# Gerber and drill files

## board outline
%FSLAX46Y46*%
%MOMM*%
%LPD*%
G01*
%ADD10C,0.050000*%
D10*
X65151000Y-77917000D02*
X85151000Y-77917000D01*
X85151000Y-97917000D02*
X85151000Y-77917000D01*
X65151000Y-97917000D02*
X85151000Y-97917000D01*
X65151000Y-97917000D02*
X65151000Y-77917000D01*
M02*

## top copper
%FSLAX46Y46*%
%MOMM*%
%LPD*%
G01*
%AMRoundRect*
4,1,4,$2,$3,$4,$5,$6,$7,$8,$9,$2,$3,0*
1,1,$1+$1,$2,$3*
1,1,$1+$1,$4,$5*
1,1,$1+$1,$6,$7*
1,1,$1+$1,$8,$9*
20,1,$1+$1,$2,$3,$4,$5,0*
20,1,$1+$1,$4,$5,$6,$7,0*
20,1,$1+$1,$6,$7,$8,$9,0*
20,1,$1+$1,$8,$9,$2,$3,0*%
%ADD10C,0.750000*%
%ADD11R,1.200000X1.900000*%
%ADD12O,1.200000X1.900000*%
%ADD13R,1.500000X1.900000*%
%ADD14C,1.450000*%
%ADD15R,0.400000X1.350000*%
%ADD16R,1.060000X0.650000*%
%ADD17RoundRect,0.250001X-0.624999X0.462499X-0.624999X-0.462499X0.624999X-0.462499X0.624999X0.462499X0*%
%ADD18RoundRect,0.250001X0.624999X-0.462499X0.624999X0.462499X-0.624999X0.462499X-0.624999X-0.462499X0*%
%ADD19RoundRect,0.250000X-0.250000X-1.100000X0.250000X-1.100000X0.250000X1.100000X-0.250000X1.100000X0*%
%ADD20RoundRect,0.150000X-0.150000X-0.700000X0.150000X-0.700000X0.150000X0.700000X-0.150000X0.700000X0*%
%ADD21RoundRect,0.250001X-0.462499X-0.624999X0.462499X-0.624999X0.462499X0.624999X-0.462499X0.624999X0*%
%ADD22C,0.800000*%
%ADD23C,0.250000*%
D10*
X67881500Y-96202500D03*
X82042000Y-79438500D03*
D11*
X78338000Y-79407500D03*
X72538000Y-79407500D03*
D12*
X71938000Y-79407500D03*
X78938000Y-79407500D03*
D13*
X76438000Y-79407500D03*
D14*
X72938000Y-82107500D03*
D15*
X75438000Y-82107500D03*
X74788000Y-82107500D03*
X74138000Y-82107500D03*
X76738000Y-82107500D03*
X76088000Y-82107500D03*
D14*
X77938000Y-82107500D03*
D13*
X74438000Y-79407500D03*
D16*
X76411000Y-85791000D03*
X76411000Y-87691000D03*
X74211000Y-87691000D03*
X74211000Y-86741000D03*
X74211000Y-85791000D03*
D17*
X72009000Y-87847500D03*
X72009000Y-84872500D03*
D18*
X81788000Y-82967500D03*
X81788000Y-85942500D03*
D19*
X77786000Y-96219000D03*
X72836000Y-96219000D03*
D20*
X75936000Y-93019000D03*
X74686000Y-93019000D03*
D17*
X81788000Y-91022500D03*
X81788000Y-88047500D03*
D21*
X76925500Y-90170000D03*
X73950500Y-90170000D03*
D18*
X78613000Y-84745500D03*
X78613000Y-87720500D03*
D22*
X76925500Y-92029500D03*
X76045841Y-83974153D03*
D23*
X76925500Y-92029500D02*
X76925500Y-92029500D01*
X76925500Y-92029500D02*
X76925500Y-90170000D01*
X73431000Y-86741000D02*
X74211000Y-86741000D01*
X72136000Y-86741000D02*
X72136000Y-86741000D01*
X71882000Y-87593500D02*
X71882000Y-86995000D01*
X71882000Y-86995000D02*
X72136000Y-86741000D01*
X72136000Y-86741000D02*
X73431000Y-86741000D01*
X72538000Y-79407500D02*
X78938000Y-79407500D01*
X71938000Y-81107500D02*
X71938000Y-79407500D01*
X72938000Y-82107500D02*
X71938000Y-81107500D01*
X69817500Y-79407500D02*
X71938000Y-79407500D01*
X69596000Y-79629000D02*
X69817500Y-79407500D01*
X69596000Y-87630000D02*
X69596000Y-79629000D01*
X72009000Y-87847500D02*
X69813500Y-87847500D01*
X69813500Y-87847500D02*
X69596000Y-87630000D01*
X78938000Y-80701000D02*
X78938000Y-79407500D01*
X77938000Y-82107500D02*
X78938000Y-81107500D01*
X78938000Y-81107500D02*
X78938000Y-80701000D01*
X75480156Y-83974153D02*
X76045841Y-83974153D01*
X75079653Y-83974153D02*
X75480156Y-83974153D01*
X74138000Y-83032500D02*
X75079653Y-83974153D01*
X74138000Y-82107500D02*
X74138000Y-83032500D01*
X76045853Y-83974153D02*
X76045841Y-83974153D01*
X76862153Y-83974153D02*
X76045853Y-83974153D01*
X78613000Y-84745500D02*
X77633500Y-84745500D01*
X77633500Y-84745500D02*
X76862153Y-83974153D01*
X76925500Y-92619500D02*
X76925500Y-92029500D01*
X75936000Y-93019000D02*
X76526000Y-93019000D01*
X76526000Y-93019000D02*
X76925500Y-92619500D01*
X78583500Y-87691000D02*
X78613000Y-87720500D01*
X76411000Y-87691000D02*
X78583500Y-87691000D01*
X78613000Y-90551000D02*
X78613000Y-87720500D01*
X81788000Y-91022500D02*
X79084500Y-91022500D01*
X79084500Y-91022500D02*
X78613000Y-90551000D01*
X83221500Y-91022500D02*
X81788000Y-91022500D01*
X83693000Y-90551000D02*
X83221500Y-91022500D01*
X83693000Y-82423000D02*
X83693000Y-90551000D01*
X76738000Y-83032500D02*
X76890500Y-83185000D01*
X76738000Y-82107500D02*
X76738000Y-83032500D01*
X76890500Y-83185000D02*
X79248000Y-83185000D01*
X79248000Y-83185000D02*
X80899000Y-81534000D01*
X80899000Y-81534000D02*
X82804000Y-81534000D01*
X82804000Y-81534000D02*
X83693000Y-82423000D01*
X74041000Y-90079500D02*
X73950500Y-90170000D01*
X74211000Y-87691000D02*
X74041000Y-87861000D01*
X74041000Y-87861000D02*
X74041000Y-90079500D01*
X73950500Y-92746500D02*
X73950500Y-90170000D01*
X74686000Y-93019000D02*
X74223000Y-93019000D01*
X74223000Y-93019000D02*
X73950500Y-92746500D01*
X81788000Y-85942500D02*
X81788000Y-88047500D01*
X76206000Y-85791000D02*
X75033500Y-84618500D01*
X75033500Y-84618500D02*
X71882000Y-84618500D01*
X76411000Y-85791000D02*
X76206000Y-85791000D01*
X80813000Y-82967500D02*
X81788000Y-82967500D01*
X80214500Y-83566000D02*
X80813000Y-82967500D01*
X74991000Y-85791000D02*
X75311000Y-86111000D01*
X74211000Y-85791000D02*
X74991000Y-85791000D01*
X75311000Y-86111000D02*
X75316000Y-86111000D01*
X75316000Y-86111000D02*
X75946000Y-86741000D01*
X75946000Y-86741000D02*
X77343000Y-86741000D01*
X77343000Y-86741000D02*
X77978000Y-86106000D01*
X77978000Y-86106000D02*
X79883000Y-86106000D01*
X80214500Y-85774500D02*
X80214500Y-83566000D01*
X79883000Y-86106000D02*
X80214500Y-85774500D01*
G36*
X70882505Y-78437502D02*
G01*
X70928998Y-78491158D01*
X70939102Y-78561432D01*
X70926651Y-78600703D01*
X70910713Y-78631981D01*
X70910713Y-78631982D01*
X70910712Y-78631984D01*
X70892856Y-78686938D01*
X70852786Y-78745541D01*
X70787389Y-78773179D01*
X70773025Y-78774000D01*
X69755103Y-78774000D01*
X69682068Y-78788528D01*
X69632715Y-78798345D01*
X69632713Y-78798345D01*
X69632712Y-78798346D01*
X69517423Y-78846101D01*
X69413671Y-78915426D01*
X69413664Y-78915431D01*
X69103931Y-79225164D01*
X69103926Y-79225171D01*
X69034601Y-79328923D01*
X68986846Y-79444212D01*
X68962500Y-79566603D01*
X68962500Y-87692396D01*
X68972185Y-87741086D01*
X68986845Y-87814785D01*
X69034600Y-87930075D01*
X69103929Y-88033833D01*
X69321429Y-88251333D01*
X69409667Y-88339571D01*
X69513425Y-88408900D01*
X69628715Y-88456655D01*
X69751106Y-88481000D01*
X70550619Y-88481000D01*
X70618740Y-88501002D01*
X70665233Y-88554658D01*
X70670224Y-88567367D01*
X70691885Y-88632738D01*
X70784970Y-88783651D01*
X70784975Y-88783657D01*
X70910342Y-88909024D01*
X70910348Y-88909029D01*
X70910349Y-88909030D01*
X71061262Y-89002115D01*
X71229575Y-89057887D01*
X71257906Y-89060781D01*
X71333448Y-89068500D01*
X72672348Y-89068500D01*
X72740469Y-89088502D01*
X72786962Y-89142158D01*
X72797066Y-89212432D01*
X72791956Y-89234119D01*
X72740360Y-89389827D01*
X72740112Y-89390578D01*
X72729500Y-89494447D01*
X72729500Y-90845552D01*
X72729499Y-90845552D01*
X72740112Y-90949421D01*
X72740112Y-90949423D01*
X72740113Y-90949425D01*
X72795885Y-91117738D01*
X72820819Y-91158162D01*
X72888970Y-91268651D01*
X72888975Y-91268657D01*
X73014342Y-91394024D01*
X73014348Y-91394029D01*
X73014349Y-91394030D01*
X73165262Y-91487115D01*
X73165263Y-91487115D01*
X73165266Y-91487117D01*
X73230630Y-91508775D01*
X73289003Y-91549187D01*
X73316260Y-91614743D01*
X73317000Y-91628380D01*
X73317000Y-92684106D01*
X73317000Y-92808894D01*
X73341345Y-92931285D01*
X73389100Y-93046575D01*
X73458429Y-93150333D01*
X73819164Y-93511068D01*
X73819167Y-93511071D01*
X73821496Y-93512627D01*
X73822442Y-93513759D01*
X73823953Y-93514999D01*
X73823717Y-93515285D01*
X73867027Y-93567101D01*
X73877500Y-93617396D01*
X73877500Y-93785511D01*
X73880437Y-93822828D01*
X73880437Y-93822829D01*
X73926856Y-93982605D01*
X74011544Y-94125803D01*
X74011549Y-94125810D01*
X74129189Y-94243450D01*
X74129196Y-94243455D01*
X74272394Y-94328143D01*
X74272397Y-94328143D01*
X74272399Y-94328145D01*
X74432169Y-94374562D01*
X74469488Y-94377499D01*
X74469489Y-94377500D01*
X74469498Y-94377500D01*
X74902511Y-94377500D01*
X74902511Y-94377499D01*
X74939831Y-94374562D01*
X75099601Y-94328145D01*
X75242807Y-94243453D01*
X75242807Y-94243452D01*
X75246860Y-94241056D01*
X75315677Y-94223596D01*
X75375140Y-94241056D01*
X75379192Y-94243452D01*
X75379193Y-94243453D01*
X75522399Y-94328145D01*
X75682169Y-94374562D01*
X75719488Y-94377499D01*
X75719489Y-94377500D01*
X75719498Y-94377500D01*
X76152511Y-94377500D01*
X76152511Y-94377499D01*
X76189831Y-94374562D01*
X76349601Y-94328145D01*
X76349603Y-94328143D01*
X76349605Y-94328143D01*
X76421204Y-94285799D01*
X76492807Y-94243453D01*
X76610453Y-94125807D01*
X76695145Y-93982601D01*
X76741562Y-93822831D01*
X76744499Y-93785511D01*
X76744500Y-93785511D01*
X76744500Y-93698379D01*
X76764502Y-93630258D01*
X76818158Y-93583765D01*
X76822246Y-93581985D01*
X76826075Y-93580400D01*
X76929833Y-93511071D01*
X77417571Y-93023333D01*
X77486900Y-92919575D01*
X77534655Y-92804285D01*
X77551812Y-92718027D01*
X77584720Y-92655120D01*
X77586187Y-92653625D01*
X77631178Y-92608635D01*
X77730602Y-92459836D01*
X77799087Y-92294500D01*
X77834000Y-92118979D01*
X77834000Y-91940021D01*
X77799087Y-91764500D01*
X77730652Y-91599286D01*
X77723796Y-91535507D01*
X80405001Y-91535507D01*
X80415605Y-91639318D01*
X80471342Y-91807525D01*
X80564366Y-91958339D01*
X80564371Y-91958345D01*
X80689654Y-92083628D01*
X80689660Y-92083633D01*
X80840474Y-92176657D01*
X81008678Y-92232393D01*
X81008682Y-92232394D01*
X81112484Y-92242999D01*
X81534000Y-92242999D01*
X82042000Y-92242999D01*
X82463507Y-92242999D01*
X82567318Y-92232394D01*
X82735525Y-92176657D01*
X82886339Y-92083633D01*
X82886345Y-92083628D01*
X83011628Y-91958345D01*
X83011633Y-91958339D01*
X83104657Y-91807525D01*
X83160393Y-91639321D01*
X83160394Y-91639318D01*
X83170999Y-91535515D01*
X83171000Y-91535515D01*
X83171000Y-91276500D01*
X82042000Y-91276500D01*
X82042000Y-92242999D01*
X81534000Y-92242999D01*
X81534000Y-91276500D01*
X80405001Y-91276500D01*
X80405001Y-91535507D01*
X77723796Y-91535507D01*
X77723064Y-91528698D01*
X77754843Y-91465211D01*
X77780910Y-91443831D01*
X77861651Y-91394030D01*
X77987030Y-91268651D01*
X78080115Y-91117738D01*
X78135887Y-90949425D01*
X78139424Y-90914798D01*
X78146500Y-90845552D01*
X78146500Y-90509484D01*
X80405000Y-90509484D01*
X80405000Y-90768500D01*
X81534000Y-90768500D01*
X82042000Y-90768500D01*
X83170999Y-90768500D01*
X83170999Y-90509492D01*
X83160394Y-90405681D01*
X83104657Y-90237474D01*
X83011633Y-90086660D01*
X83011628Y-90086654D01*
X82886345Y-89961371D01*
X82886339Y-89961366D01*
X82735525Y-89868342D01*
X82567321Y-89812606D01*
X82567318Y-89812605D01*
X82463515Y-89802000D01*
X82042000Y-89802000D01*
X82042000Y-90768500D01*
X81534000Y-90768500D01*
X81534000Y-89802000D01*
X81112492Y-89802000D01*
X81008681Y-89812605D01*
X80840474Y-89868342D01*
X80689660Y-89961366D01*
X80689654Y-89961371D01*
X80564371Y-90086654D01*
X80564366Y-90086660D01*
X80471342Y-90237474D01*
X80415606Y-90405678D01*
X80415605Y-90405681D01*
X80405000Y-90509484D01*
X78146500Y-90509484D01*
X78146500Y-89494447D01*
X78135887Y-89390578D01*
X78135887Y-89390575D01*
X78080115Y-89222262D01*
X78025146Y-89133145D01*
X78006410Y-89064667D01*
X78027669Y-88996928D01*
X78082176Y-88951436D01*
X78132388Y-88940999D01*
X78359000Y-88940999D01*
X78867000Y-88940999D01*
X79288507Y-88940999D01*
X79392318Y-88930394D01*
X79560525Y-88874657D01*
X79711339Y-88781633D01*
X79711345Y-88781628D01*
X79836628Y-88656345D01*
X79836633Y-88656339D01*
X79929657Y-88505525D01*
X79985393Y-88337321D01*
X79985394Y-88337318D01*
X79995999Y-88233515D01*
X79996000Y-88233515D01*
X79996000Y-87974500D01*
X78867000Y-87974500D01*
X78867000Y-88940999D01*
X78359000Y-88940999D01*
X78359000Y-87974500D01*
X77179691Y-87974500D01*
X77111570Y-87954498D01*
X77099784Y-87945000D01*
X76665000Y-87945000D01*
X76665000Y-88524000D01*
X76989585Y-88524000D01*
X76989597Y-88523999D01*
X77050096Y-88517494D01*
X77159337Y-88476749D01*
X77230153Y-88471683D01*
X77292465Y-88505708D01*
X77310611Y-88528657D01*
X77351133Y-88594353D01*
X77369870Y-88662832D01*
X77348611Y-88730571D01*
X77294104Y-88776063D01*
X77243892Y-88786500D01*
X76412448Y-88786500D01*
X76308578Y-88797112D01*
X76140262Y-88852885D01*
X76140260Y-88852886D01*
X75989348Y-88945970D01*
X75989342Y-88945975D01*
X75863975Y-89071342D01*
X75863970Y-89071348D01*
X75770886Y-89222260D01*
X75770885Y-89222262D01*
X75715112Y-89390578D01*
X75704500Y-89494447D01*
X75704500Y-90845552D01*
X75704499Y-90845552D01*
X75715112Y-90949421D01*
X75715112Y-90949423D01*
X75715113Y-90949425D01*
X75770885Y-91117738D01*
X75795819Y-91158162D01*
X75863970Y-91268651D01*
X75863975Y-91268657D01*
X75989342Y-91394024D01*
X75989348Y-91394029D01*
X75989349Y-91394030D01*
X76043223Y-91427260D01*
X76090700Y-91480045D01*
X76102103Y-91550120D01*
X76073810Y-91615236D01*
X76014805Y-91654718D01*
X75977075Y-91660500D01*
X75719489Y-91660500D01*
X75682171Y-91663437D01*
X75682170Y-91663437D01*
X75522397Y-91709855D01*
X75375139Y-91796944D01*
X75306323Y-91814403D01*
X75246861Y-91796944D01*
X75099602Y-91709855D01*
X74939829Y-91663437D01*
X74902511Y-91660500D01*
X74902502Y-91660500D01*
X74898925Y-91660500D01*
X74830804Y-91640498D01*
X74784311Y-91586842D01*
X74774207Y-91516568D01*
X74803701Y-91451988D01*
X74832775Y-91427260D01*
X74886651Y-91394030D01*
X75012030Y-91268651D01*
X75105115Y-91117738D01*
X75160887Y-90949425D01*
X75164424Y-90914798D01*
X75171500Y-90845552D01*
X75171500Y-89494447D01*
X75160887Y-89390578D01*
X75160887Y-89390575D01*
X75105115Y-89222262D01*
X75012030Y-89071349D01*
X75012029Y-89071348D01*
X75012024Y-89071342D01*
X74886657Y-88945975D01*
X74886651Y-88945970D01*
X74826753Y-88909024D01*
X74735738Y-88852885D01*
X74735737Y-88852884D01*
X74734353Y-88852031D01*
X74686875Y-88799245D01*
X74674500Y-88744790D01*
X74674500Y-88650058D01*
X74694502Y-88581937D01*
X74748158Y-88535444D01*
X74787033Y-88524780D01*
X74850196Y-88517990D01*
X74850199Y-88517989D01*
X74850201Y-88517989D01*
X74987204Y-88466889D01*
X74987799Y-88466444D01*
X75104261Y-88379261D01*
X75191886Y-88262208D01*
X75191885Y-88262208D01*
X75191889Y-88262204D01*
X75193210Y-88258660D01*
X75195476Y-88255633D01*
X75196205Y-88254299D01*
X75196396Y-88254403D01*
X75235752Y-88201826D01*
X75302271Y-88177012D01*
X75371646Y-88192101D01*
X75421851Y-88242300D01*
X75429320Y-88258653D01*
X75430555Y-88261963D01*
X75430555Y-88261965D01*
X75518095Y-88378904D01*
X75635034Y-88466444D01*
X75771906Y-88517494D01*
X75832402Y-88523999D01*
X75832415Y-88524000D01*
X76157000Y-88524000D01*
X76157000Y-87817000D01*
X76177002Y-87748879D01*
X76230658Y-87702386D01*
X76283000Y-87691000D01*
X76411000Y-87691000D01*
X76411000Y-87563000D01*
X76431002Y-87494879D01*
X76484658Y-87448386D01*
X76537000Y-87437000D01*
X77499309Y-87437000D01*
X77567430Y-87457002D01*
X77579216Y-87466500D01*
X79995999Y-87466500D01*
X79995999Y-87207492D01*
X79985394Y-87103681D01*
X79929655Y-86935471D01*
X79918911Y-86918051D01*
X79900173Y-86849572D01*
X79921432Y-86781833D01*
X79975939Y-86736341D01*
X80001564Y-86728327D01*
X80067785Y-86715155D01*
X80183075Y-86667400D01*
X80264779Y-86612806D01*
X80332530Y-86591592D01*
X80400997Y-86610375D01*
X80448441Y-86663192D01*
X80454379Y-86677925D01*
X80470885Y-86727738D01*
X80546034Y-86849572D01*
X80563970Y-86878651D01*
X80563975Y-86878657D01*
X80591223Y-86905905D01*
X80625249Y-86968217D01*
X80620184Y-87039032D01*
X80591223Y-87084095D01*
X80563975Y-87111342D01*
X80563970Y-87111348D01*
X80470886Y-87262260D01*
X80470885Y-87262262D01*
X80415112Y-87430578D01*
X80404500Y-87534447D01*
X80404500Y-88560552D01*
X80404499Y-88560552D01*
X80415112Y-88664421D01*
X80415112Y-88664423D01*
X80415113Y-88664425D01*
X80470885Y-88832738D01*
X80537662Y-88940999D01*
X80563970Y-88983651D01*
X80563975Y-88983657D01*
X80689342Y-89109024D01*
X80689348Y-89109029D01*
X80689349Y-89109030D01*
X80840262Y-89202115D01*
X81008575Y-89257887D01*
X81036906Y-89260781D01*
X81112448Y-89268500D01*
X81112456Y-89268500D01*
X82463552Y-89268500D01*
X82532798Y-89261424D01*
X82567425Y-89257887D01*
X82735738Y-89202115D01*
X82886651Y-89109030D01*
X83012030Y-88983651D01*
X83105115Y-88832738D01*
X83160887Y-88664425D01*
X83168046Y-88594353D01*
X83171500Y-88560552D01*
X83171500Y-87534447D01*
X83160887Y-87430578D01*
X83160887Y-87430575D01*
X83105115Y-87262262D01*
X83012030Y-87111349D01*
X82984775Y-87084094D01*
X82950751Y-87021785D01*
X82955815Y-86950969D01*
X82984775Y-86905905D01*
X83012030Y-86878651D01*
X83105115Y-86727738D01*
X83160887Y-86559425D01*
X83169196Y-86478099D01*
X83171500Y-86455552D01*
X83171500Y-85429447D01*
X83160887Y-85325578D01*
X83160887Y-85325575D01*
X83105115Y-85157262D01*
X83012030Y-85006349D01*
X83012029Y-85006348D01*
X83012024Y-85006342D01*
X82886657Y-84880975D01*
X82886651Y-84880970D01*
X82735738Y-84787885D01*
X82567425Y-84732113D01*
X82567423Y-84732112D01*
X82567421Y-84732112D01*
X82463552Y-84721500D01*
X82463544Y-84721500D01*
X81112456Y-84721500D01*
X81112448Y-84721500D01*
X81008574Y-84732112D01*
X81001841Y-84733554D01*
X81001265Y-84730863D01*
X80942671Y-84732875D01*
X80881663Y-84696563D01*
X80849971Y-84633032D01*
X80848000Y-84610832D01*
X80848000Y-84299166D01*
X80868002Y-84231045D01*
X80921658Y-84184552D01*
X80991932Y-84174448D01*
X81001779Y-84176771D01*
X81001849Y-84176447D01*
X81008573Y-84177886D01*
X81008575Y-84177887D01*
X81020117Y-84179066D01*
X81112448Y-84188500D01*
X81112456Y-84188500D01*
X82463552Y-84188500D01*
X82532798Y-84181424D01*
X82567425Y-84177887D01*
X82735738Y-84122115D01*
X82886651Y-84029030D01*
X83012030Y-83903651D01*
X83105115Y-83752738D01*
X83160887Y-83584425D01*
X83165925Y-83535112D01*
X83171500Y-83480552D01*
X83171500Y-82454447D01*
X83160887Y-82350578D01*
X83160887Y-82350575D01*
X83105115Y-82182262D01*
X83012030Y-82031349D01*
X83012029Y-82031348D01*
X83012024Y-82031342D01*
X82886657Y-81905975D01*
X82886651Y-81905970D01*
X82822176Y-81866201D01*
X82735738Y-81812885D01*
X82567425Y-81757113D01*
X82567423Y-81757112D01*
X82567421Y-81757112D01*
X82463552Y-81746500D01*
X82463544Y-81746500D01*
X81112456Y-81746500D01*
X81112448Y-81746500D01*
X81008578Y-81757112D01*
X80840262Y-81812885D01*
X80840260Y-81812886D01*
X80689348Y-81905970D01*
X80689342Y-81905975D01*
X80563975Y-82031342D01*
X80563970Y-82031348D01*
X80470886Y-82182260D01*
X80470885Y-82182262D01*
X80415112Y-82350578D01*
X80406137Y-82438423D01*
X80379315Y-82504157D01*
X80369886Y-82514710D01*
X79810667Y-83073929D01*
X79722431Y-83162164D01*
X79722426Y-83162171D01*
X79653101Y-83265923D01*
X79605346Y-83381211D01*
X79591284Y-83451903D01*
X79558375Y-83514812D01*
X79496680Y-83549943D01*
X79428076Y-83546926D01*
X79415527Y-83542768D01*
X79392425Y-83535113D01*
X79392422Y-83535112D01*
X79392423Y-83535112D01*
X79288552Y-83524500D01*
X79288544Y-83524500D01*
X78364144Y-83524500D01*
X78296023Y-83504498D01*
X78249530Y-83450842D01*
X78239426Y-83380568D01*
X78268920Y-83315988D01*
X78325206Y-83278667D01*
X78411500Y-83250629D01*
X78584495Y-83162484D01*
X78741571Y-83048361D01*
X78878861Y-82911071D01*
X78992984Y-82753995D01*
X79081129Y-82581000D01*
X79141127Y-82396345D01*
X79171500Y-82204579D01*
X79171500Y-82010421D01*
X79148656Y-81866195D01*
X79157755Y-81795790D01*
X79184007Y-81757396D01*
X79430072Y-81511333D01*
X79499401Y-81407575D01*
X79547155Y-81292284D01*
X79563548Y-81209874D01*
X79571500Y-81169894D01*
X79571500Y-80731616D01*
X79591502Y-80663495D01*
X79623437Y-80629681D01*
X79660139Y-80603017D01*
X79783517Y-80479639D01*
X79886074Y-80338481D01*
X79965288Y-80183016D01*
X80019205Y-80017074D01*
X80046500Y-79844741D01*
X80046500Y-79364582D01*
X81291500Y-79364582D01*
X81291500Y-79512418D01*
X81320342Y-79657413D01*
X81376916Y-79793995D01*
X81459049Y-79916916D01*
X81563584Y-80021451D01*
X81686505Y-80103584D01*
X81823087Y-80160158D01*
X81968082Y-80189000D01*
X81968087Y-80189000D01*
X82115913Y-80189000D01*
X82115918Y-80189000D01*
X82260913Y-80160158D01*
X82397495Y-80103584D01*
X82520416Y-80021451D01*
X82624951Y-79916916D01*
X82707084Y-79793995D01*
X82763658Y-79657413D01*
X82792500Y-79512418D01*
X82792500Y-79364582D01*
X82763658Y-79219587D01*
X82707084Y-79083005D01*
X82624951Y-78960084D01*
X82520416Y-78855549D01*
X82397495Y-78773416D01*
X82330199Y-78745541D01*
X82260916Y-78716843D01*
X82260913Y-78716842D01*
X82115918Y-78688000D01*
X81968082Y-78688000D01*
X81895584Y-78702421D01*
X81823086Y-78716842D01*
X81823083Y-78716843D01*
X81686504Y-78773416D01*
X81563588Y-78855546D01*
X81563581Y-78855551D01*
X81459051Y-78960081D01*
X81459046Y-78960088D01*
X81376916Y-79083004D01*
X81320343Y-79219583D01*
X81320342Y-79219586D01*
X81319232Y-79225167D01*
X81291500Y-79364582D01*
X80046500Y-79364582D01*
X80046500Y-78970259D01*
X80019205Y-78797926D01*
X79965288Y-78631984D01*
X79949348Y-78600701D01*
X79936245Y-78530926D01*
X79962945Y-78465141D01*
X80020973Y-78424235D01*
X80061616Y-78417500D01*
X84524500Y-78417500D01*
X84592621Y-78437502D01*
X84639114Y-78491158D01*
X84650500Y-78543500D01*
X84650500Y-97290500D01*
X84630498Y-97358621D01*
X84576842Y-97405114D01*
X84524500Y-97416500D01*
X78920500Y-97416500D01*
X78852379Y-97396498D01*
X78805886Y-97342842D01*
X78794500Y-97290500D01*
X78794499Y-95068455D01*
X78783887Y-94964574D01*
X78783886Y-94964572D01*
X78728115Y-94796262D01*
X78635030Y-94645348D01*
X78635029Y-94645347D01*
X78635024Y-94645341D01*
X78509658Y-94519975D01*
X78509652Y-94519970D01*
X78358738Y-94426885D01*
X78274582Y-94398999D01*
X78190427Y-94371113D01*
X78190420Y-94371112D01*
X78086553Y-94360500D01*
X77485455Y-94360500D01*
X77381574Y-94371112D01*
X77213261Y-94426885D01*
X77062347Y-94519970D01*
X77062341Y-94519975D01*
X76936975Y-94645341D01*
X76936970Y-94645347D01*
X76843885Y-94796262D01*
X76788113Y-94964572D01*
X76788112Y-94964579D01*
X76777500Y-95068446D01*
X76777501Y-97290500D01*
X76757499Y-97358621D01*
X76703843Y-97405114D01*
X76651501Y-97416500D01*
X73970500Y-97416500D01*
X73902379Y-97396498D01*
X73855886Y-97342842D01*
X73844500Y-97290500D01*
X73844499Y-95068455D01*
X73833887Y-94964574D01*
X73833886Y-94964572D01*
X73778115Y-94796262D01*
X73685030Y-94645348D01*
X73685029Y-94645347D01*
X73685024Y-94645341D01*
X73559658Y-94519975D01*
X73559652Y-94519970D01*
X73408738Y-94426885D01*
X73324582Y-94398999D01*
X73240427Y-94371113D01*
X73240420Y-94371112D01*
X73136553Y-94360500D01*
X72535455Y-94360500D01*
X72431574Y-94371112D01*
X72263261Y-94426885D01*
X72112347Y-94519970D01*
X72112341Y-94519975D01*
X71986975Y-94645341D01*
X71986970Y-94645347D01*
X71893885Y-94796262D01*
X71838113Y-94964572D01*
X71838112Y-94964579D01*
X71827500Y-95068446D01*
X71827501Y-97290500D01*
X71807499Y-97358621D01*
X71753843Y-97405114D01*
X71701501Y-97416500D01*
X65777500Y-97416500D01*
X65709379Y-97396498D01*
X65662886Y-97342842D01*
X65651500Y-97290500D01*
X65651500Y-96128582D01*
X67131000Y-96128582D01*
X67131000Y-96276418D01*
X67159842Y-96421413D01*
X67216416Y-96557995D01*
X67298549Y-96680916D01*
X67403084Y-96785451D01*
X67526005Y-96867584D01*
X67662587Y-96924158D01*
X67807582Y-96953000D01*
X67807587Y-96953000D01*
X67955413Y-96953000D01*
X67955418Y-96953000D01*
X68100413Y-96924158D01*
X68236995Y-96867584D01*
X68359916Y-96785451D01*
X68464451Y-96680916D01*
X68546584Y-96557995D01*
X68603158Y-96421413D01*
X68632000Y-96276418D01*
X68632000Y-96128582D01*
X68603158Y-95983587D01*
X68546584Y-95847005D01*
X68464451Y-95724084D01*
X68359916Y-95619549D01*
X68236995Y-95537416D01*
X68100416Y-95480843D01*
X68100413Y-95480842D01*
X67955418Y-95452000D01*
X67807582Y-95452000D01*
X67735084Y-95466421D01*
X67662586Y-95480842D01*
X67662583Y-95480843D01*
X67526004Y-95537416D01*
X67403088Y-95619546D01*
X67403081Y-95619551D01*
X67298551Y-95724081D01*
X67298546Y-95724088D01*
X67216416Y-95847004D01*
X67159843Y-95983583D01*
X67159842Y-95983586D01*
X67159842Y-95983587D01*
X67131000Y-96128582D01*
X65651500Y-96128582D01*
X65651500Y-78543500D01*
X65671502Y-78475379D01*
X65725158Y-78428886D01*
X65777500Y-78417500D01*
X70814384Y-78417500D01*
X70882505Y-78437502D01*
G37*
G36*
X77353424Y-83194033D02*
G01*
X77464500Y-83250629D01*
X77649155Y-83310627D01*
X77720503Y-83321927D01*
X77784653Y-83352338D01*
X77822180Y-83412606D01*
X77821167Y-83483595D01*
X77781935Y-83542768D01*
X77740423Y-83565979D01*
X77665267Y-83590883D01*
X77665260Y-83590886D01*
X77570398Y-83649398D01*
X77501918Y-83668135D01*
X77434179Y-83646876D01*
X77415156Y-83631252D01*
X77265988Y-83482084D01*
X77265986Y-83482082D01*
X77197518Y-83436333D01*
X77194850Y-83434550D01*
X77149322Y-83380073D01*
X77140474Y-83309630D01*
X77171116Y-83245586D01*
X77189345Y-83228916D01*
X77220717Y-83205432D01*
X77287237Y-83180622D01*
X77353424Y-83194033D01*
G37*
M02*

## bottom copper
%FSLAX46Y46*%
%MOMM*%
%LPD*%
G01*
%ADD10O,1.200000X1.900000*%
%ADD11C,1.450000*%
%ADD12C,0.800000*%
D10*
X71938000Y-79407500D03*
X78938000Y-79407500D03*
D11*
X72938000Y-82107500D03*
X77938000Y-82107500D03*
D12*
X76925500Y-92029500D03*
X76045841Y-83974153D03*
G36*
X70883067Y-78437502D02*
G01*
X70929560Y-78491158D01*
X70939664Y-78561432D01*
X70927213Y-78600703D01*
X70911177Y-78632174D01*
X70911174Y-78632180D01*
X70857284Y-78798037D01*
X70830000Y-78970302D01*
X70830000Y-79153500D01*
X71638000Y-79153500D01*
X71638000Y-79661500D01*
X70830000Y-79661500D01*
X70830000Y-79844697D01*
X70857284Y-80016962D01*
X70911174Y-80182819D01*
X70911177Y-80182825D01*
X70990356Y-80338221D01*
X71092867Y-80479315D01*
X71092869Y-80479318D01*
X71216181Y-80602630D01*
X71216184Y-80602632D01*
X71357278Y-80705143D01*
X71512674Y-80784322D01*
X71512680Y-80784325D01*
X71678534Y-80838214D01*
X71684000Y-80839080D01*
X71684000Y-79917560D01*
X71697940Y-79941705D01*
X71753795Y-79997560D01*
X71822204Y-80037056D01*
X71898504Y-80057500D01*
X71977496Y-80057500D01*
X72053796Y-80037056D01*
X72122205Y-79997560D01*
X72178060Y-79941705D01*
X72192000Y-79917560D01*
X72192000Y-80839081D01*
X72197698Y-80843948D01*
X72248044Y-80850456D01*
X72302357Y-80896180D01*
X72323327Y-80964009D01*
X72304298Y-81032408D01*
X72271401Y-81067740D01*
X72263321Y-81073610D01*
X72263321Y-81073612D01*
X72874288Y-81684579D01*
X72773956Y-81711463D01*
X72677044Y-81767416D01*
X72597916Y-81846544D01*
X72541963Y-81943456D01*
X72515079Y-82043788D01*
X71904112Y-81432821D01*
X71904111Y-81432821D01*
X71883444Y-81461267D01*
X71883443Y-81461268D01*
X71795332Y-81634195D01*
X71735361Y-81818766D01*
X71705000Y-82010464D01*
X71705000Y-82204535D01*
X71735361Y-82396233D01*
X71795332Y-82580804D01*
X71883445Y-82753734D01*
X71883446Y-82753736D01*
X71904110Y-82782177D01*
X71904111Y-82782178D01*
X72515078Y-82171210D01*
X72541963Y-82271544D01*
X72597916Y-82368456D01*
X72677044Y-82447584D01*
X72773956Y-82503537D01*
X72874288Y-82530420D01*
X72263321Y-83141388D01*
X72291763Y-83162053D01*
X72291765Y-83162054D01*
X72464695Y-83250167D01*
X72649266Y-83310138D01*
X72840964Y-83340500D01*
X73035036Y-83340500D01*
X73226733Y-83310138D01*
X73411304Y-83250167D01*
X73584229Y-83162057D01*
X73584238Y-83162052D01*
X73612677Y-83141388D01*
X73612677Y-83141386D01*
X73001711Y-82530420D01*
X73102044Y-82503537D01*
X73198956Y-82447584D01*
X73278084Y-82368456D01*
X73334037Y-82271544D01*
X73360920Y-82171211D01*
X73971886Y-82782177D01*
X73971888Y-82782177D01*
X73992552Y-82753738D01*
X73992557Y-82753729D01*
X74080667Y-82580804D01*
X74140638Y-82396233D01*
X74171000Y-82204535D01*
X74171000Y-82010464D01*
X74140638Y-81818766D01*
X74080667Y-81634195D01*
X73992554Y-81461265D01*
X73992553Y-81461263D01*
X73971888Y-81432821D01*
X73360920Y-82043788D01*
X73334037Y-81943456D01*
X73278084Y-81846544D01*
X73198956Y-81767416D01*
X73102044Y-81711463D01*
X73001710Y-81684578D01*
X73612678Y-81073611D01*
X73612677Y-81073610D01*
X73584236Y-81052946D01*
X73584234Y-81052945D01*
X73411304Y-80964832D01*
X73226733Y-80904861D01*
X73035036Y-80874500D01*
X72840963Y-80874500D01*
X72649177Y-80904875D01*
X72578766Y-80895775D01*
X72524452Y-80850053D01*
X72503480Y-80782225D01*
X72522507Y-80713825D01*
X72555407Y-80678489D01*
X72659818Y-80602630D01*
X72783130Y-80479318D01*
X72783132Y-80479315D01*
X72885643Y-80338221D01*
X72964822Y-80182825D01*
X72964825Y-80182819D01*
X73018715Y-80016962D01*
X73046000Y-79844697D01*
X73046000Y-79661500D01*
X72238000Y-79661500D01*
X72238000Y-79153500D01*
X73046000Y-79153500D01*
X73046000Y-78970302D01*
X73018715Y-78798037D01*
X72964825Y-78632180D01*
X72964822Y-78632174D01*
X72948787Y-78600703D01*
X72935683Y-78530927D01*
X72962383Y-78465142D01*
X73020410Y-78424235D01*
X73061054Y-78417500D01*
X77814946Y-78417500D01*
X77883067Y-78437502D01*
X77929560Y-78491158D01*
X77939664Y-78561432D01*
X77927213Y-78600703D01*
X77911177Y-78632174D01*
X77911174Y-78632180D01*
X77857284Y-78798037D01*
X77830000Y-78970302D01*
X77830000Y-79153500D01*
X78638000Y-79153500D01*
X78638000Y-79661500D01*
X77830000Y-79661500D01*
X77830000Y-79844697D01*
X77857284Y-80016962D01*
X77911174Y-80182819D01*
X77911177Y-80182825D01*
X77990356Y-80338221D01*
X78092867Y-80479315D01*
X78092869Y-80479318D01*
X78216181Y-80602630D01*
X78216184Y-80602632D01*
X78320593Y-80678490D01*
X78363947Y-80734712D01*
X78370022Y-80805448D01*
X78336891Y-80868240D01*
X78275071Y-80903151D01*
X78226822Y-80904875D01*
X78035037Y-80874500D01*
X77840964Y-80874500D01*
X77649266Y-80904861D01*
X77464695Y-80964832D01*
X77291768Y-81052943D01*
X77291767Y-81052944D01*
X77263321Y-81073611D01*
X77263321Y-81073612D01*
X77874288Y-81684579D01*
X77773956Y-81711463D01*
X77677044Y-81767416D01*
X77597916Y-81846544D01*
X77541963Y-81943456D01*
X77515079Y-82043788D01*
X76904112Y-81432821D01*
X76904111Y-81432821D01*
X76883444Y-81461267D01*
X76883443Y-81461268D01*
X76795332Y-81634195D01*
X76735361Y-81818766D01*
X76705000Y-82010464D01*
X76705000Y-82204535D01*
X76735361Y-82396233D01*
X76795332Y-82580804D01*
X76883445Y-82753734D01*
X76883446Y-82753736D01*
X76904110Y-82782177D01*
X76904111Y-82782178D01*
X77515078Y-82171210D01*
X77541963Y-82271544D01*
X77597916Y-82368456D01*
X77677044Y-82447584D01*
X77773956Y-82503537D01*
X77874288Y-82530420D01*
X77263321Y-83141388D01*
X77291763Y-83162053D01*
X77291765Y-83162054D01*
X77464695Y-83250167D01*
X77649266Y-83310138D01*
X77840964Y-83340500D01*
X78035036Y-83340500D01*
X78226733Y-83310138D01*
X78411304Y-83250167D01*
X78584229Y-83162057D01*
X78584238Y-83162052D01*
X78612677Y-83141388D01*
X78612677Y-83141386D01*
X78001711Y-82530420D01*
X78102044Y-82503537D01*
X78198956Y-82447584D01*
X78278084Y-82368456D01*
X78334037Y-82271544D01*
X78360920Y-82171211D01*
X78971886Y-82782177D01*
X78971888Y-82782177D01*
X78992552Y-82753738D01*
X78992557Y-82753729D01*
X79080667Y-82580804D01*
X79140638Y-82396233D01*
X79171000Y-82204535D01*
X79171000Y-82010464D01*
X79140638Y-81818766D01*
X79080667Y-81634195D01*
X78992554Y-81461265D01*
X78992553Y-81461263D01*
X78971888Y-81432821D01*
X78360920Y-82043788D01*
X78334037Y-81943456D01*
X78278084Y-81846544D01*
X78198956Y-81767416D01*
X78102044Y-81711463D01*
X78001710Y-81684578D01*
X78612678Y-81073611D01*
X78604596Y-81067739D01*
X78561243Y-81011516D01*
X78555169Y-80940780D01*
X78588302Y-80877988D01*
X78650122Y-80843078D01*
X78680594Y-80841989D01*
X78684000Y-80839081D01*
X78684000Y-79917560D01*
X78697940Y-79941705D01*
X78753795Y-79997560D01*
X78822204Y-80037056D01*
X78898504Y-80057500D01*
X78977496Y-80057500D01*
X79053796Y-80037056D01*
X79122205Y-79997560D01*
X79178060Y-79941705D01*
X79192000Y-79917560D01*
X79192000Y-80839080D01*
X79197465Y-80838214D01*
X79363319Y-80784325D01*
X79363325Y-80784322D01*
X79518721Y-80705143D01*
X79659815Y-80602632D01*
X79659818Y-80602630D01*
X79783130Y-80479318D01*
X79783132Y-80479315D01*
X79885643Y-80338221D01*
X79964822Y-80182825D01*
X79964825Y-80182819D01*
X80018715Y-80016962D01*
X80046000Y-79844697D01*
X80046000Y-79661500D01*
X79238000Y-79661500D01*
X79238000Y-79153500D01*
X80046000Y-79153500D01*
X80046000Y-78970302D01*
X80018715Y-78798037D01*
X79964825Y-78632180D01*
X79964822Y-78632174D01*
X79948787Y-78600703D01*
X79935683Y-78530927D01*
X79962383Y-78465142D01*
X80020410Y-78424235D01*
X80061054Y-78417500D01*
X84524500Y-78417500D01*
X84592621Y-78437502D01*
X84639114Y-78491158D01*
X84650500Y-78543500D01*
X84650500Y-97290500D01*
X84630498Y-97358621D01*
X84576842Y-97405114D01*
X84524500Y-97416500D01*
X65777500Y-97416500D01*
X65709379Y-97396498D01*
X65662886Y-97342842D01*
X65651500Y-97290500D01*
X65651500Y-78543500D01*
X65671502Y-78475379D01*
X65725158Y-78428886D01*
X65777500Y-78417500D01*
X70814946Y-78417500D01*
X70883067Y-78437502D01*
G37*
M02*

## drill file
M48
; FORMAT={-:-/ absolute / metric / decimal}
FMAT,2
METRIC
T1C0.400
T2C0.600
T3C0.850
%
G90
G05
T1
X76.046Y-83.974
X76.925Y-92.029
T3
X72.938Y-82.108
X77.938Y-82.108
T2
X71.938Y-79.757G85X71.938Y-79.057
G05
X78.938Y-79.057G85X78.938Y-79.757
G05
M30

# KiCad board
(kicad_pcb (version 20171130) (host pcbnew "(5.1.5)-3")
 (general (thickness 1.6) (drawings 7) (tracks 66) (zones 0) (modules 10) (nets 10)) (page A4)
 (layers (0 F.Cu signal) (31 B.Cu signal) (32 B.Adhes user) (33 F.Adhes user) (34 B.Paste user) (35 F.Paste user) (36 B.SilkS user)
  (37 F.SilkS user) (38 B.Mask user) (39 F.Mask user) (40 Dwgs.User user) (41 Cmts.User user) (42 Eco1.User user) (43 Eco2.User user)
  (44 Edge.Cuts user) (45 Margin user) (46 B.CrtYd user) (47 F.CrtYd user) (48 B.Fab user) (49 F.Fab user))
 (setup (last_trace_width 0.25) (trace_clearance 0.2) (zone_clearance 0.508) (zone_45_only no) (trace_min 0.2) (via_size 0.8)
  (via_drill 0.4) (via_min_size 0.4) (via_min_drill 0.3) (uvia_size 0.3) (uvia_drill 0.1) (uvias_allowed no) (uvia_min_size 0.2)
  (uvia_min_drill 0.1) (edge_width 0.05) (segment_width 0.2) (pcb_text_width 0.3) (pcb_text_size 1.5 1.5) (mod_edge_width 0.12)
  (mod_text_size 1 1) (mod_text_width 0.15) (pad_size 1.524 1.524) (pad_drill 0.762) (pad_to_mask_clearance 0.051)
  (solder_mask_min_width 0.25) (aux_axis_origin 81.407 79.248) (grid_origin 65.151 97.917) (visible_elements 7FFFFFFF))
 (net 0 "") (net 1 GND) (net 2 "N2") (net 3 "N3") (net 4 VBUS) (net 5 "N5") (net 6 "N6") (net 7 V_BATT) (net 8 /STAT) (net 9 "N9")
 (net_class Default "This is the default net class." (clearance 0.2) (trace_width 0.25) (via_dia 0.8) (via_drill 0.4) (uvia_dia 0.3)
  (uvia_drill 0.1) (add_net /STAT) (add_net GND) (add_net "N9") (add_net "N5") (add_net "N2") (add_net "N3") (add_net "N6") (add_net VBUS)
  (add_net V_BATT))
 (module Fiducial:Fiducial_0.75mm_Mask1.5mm (layer F.Cu) (at 67.8815 96.2025)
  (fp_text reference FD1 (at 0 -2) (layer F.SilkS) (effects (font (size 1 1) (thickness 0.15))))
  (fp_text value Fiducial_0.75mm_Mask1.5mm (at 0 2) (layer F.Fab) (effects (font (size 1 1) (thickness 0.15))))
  (pad "" smd circle (at 0 0) (size 0.75 0.75) (layers F.Cu F.Mask) (solder_mask_margin 0.375) (clearance 0.375)))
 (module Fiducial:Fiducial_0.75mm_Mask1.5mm (layer F.Cu) (at 82.042 79.4385)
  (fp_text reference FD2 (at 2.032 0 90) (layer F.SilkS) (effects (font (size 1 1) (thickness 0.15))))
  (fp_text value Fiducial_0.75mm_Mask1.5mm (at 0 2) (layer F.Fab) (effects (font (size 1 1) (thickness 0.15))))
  (pad "" smd circle (at 0 0) (size 0.75 0.75) (layers F.Cu F.Mask) (solder_mask_margin 0.375) (clearance 0.375)))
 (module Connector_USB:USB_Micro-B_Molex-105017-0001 (layer F.Cu) (at 75.438 80.645 180)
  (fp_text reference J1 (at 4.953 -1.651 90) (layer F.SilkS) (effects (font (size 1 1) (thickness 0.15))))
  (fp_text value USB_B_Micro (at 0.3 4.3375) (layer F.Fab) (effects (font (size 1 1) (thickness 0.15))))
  (pad 6 smd rect (at -2.9 1.2375 180) (size 1.2 1.9) (layers F.Cu F.Mask) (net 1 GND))
  (pad 6 smd rect (at 2.9 1.2375 180) (size 1.2 1.9) (layers F.Cu F.Mask) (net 1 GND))
  (pad 6 thru_hole oval (at 3.5 1.2375 180) (size 1.2 1.9) (drill oval 0.6 1.3) (layers *.Cu *.Mask) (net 1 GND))
  (pad 6 thru_hole oval (at -3.5 1.2375) (size 1.2 1.9) (drill oval 0.6 1.3) (layers *.Cu *.Mask) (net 1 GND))
  (pad 6 smd rect (at -1 1.2375 180) (size 1.5 1.9) (layers F.Cu F.Paste F.Mask) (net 1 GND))
  (pad 6 thru_hole circle (at 2.5 -1.4625 180) (size 1.45 1.45) (drill 0.85) (layers *.Cu *.Mask) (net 1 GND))
  (pad 3 smd rect (at 0 -1.4625 180) (size 0.4 1.35) (layers F.Cu F.Paste F.Mask) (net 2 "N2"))
  (pad 4 smd rect (at 0.65 -1.4625 180) (size 0.4 1.35) (layers F.Cu F.Paste F.Mask) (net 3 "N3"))
  (pad 5 smd rect (at 1.3 -1.4625 180) (size 0.4 1.35) (layers F.Cu F.Paste F.Mask) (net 1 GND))
  (pad 1 smd rect (at -1.3 -1.4625 180) (size 0.4 1.35) (layers F.Cu F.Paste F.Mask) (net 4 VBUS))
  (pad 2 smd rect (at -0.65 -1.4625 180) (size 0.4 1.35) (layers F.Cu F.Paste F.Mask) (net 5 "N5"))
  (pad 6 thru_hole circle (at -2.5 -1.4625 180) (size 1.45 1.45) (drill 0.85) (layers *.Cu *.Mask) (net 1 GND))
  (pad 6 smd rect (at 1 1.2375 180) (size 1.5 1.9) (layers F.Cu F.Paste F.Mask) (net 1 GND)))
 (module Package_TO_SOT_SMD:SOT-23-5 (layer F.Cu) (at 75.311 86.741)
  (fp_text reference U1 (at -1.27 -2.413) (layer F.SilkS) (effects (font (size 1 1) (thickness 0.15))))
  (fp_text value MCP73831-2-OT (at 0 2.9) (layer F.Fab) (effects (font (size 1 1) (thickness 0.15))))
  (pad 5 smd rect (at 1.1 -0.95) (size 1.06 0.65) (layers F.Cu F.Paste F.Mask) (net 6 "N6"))
  (pad 4 smd rect (at 1.1 0.95) (size 1.06 0.65) (layers F.Cu F.Paste F.Mask) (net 4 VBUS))
  (pad 3 smd rect (at -1.1 0.95) (size 1.06 0.65) (layers F.Cu F.Paste F.Mask) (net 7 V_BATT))
  (pad 2 smd rect (at -1.1 0) (size 1.06 0.65) (layers F.Cu F.Paste F.Mask) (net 1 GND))
  (pad 1 smd rect (at -1.1 -0.95) (size 1.06 0.65) (layers F.Cu F.Paste F.Mask) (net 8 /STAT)))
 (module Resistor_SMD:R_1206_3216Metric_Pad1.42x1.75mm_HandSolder (layer F.Cu) (at 72.009 86.36 270)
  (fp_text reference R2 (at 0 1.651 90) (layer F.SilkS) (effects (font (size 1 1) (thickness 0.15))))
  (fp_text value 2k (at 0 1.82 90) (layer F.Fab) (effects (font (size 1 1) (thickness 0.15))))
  (pad 2 smd roundrect (at 1.4875 0 270) (size 1.425 1.75) (layers F.Cu F.Paste F.Mask) (roundrect_rratio 0.175439) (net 1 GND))
  (pad 1 smd roundrect (at -1.4875 0 270) (size 1.425 1.75) (layers F.Cu F.Paste F.Mask) (roundrect_rratio 0.175439) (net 6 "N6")))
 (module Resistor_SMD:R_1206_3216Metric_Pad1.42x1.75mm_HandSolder (layer F.Cu) (at 81.788 84.455 90)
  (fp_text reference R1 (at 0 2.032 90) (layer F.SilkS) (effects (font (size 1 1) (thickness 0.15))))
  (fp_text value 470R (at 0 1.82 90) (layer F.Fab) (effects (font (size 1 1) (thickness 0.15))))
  (pad 2 smd roundrect (at 1.4875 0 90) (size 1.425 1.75) (layers F.Cu F.Paste F.Mask) (roundrect_rratio 0.175439) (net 8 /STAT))
  (pad 1 smd roundrect (at -1.4875 0 90) (size 1.425 1.75) (layers F.Cu F.Paste F.Mask) (roundrect_rratio 0.175439) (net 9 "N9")))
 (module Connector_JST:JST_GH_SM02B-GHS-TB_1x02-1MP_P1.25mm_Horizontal (layer F.Cu) (at 75.311 94.869)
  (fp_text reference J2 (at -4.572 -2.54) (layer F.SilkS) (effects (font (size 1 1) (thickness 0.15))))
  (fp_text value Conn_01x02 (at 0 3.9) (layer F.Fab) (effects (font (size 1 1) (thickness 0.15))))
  (pad MP smd roundrect (at 2.475 1.35) (size 1 2.7) (layers F.Cu F.Paste F.Mask) (roundrect_rratio 0.25))
  (pad MP smd roundrect (at -2.475 1.35) (size 1 2.7) (layers F.Cu F.Paste F.Mask) (roundrect_rratio 0.25))
  (pad 2 smd roundrect (at 0.625 -1.85) (size 0.6 1.7) (layers F.Cu F.Paste F.Mask) (roundrect_rratio 0.25) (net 1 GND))
  (pad 1 smd roundrect (at -0.625 -1.85) (size 0.6 1.7) (layers F.Cu F.Paste F.Mask) (roundrect_rratio 0.25) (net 7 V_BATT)))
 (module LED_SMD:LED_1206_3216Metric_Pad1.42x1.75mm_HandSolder (layer F.Cu) (at 81.788 89.535 270)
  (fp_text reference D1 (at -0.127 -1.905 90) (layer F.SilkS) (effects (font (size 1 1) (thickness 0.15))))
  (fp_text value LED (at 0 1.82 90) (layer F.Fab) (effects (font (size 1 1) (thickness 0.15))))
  (pad 2 smd roundrect (at 1.4875 0 270) (size 1.425 1.75) (layers F.Cu F.Paste F.Mask) (roundrect_rratio 0.175439) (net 4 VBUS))
  (pad 1 smd roundrect (at -1.4875 0 270) (size 1.425 1.75) (layers F.Cu F.Paste F.Mask) (roundrect_rratio 0.175439) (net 9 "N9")))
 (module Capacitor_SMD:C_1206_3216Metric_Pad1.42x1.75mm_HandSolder (layer F.Cu) (at 75.438 90.17)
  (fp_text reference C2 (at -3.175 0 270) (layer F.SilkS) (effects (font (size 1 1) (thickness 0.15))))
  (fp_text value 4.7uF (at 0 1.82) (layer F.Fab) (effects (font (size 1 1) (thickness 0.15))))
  (pad 2 smd roundrect (at 1.4875 0) (size 1.425 1.75) (layers F.Cu F.Paste F.Mask) (roundrect_rratio 0.175439) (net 1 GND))
  (pad 1 smd roundrect (at -1.4875 0) (size 1.425 1.75) (layers F.Cu F.Paste F.Mask) (roundrect_rratio 0.175439) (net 7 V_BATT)))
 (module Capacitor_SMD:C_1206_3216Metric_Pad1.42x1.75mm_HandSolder (layer F.Cu) (at 78.613 86.233 90)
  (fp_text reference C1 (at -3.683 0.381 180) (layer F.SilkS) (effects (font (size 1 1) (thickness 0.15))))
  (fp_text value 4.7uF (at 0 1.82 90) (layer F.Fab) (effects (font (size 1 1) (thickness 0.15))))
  (pad 2 smd roundrect (at 1.4875 0 90) (size 1.425 1.75) (layers F.Cu F.Paste F.Mask) (roundrect_rratio 0.175439) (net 1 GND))
  (pad 1 smd roundrect (at -1.4875 0 90) (size 1.425 1.75) (layers F.Cu F.Paste F.Mask) (roundrect_rratio 0.175439) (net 4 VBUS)))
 (gr_line (start 65.151 77.917) (end 85.151 77.917) (layer Edge.Cuts) (width 0.05))
 (gr_line (start 85.151 97.917) (end 85.151 77.917) (layer Edge.Cuts) (width 0.05))
 (gr_line (start 65.151 97.917) (end 85.151 97.917) (layer Edge.Cuts) (width 0.05))
 (gr_line (start 65.151 97.917) (end 65.151 77.917) (layer Edge.Cuts) (width 0.05))
 (segment (start 76.9255 92.0295) (end 76.9255 92.0295) (width 0.25) (layer F.Cu) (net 1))
 (segment (start 76.9255 92.0295) (end 76.9255 90.17) (width 0.25) (layer F.Cu) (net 1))
 (via (at 76.9255 92.0295) (size 0.8) (drill 0.4) (layers F.Cu B.Cu) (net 1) (status 1000000))
 (segment (start 73.431 86.741) (end 74.211 86.741) (width 0.25) (layer F.Cu) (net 1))
 (segment (start 72.136 86.741) (end 72.136 86.741) (width 0.25) (layer F.Cu) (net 1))
 (segment (start 71.882 87.5935) (end 71.882 86.995) (width 0.25) (layer F.Cu) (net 1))
 (segment (start 71.882 86.995) (end 72.136 86.741) (width 0.25) (layer F.Cu) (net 1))
 (segment (start 72.136 86.741) (end 73.431 86.741) (width 0.25) (layer F.Cu) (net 1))
 (segment (start 72.538 79.4075) (end 78.938 79.4075) (width 0.25) (layer F.Cu) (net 1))
 (segment (start 71.938 81.1075) (end 71.938 79.4075) (width 0.25) (layer F.Cu) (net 1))
 (segment (start 72.938 82.1075) (end 71.938 81.1075) (width 0.25) (layer F.Cu) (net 1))
 (segment (start 69.8175 79.4075) (end 71.938 79.4075) (width 0.25) (layer F.Cu) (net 1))
 (segment (start 69.596 79.629) (end 69.8175 79.4075) (width 0.25) (layer F.Cu) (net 1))
 (segment (start 69.596 87.63) (end 69.596 79.629) (width 0.25) (layer F.Cu) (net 1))
 (segment (start 72.009 87.8475) (end 69.8135 87.8475) (width 0.25) (layer F.Cu) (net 1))
 (segment (start 69.8135 87.8475) (end 69.596 87.63) (width 0.25) (layer F.Cu) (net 1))
 (segment (start 78.938 80.701) (end 78.938 79.4075) (width 0.25) (layer F.Cu) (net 1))
 (segment (start 77.938 82.1075) (end 78.938 81.1075) (width 0.25) (layer F.Cu) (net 1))
 (segment (start 78.938 81.1075) (end 78.938 80.701) (width 0.25) (layer F.Cu) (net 1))
 (via (at 76.045841 83.974153) (size 0.8) (drill 0.4) (layers F.Cu B.Cu) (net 1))
 (segment (start 75.480156 83.974153) (end 76.045841 83.974153) (width 0.25) (layer F.Cu) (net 1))
 (segment (start 75.079653 83.974153) (end 75.480156 83.974153) (width 0.25) (layer F.Cu) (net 1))
 (segment (start 74.138 83.0325) (end 75.079653 83.974153) (width 0.25) (layer F.Cu) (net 1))
 (segment (start 74.138 82.1075) (end 74.138 83.0325) (width 0.25) (layer F.Cu) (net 1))
 (segment (start 76.045853 83.974153) (end 76.045841 83.974153) (width 0.25) (layer F.Cu) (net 1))
 (segment (start 76.862153 83.974153) (end 76.045853 83.974153) (width 0.25) (layer F.Cu) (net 1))
 (segment (start 78.613 84.7455) (end 77.6335 84.7455) (width 0.25) (layer F.Cu) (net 1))
 (segment (start 77.6335 84.7455) (end 76.862153 83.974153) (width 0.25) (layer F.Cu) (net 1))
 (segment (start 76.9255 92.6195) (end 76.9255 92.0295) (width 0.25) (layer F.Cu) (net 1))
 (segment (start 75.936 93.019) (end 76.526 93.019) (width 0.25) (layer F.Cu) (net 1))
 (segment (start 76.526 93.019) (end 76.9255 92.6195) (width 0.25) (layer F.Cu) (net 1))
 (segment (start 78.5835 87.691) (end 78.613 87.7205) (width 0.25) (layer F.Cu) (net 4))
 (segment (start 76.411 87.691) (end 78.5835 87.691) (width 0.25) (layer F.Cu) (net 4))
 (segment (start 78.613 90.551) (end 78.613 87.7205) (width 0.25) (layer F.Cu) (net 4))
 (segment (start 81.788 91.0225) (end 79.0845 91.0225) (width 0.25) (layer F.Cu) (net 4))
 (segment (start 79.0845 91.0225) (end 78.613 90.551) (width 0.25) (layer F.Cu) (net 4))
 (segment (start 83.2215 91.0225) (end 81.788 91.0225) (width 0.25) (layer F.Cu) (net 4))
 (segment (start 83.693 90.551) (end 83.2215 91.0225) (width 0.25) (layer F.Cu) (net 4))
 (segment (start 83.693 82.423) (end 83.693 90.551) (width 0.25) (layer F.Cu) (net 4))
 (segment (start 76.738 83.0325) (end 76.8905 83.185) (width 0.25) (layer F.Cu) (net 4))
 (segment (start 76.738 82.1075) (end 76.738 83.0325) (width 0.25) (layer F.Cu) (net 4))
 (segment (start 76.8905 83.185) (end 79.248 83.185) (width 0.25) (layer F.Cu) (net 4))
 (segment (start 79.248 83.185) (end 80.899 81.534) (width 0.25) (layer F.Cu) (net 4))
 (segment (start 80.899 81.534) (end 82.804 81.534) (width 0.25) (layer F.Cu) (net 4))
 (segment (start 82.804 81.534) (end 83.693 82.423) (width 0.25) (layer F.Cu) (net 4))
 (segment (start 74.041 90.0795) (end 73.9505 90.17) (width 0.25) (layer F.Cu) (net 7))
 (segment (start 74.211 87.691) (end 74.041 87.861) (width 0.25) (layer F.Cu) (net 7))
 (segment (start 74.041 87.861) (end 74.041 90.0795) (width 0.25) (layer F.Cu) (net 7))
 (segment (start 73.9505 92.7465) (end 73.9505 90.17) (width 0.25) (layer F.Cu) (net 7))
 (segment (start 74.686 93.019) (end 74.223 93.019) (width 0.25) (layer F.Cu) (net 7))
 (segment (start 74.223 93.019) (end 73.9505 92.7465) (width 0.25) (layer F.Cu) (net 7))
 (segment (start 81.788 85.9425) (end 81.788 88.0475) (width 0.25) (layer F.Cu) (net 9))
 (segment (start 76.206 85.791) (end 75.0335 84.6185) (width 0.25) (layer F.Cu) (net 6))
 (segment (start 75.0335 84.6185) (end 71.882 84.6185) (width 0.25) (layer F.Cu) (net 6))
 (segment (start 76.411 85.791) (end 76.206 85.791) (width 0.25) (layer F.Cu) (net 6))
 (segment (start 80.813 82.9675) (end 81.788 82.9675) (width 0.25) (layer F.Cu) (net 8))
 (segment (start 80.2145 83.566) (end 80.813 82.9675) (width 0.25) (layer F.Cu) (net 8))
 (segment (start 74.991 85.791) (end 75.311 86.111) (width 0.25) (layer F.Cu) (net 8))
 (segment (start 74.211 85.791) (end 74.991 85.791) (width 0.25) (layer F.Cu) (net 8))
 (segment (start 75.311 86.111) (end 75.316 86.111) (width 0.25) (layer F.Cu) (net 8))
 (segment (start 75.316 86.111) (end 75.946 86.741) (width 0.25) (layer F.Cu) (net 8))
 (segment (start 75.946 86.741) (end 77.343 86.741) (width 0.25) (layer F.Cu) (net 8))
 (segment (start 77.343 86.741) (end 77.978 86.106) (width 0.25) (layer F.Cu) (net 8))
 (segment (start 77.978 86.106) (end 79.883 86.106) (width 0.25) (layer F.Cu) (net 8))
 (segment (start 80.2145 85.7745) (end 80.2145 83.566) (width 0.25) (layer F.Cu) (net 8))
 (segment (start 79.883 86.106) (end 80.2145 85.7745) (width 0.25) (layer F.Cu) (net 8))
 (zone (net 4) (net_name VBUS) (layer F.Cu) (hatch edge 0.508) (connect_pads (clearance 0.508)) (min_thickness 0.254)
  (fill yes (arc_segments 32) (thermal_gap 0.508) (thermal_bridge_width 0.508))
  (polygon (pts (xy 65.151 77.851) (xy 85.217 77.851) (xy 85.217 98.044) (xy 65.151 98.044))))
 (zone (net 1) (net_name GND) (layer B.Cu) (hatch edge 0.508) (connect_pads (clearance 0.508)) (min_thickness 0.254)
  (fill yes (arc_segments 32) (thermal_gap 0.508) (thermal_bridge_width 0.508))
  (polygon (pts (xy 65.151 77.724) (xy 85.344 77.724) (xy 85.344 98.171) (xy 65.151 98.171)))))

